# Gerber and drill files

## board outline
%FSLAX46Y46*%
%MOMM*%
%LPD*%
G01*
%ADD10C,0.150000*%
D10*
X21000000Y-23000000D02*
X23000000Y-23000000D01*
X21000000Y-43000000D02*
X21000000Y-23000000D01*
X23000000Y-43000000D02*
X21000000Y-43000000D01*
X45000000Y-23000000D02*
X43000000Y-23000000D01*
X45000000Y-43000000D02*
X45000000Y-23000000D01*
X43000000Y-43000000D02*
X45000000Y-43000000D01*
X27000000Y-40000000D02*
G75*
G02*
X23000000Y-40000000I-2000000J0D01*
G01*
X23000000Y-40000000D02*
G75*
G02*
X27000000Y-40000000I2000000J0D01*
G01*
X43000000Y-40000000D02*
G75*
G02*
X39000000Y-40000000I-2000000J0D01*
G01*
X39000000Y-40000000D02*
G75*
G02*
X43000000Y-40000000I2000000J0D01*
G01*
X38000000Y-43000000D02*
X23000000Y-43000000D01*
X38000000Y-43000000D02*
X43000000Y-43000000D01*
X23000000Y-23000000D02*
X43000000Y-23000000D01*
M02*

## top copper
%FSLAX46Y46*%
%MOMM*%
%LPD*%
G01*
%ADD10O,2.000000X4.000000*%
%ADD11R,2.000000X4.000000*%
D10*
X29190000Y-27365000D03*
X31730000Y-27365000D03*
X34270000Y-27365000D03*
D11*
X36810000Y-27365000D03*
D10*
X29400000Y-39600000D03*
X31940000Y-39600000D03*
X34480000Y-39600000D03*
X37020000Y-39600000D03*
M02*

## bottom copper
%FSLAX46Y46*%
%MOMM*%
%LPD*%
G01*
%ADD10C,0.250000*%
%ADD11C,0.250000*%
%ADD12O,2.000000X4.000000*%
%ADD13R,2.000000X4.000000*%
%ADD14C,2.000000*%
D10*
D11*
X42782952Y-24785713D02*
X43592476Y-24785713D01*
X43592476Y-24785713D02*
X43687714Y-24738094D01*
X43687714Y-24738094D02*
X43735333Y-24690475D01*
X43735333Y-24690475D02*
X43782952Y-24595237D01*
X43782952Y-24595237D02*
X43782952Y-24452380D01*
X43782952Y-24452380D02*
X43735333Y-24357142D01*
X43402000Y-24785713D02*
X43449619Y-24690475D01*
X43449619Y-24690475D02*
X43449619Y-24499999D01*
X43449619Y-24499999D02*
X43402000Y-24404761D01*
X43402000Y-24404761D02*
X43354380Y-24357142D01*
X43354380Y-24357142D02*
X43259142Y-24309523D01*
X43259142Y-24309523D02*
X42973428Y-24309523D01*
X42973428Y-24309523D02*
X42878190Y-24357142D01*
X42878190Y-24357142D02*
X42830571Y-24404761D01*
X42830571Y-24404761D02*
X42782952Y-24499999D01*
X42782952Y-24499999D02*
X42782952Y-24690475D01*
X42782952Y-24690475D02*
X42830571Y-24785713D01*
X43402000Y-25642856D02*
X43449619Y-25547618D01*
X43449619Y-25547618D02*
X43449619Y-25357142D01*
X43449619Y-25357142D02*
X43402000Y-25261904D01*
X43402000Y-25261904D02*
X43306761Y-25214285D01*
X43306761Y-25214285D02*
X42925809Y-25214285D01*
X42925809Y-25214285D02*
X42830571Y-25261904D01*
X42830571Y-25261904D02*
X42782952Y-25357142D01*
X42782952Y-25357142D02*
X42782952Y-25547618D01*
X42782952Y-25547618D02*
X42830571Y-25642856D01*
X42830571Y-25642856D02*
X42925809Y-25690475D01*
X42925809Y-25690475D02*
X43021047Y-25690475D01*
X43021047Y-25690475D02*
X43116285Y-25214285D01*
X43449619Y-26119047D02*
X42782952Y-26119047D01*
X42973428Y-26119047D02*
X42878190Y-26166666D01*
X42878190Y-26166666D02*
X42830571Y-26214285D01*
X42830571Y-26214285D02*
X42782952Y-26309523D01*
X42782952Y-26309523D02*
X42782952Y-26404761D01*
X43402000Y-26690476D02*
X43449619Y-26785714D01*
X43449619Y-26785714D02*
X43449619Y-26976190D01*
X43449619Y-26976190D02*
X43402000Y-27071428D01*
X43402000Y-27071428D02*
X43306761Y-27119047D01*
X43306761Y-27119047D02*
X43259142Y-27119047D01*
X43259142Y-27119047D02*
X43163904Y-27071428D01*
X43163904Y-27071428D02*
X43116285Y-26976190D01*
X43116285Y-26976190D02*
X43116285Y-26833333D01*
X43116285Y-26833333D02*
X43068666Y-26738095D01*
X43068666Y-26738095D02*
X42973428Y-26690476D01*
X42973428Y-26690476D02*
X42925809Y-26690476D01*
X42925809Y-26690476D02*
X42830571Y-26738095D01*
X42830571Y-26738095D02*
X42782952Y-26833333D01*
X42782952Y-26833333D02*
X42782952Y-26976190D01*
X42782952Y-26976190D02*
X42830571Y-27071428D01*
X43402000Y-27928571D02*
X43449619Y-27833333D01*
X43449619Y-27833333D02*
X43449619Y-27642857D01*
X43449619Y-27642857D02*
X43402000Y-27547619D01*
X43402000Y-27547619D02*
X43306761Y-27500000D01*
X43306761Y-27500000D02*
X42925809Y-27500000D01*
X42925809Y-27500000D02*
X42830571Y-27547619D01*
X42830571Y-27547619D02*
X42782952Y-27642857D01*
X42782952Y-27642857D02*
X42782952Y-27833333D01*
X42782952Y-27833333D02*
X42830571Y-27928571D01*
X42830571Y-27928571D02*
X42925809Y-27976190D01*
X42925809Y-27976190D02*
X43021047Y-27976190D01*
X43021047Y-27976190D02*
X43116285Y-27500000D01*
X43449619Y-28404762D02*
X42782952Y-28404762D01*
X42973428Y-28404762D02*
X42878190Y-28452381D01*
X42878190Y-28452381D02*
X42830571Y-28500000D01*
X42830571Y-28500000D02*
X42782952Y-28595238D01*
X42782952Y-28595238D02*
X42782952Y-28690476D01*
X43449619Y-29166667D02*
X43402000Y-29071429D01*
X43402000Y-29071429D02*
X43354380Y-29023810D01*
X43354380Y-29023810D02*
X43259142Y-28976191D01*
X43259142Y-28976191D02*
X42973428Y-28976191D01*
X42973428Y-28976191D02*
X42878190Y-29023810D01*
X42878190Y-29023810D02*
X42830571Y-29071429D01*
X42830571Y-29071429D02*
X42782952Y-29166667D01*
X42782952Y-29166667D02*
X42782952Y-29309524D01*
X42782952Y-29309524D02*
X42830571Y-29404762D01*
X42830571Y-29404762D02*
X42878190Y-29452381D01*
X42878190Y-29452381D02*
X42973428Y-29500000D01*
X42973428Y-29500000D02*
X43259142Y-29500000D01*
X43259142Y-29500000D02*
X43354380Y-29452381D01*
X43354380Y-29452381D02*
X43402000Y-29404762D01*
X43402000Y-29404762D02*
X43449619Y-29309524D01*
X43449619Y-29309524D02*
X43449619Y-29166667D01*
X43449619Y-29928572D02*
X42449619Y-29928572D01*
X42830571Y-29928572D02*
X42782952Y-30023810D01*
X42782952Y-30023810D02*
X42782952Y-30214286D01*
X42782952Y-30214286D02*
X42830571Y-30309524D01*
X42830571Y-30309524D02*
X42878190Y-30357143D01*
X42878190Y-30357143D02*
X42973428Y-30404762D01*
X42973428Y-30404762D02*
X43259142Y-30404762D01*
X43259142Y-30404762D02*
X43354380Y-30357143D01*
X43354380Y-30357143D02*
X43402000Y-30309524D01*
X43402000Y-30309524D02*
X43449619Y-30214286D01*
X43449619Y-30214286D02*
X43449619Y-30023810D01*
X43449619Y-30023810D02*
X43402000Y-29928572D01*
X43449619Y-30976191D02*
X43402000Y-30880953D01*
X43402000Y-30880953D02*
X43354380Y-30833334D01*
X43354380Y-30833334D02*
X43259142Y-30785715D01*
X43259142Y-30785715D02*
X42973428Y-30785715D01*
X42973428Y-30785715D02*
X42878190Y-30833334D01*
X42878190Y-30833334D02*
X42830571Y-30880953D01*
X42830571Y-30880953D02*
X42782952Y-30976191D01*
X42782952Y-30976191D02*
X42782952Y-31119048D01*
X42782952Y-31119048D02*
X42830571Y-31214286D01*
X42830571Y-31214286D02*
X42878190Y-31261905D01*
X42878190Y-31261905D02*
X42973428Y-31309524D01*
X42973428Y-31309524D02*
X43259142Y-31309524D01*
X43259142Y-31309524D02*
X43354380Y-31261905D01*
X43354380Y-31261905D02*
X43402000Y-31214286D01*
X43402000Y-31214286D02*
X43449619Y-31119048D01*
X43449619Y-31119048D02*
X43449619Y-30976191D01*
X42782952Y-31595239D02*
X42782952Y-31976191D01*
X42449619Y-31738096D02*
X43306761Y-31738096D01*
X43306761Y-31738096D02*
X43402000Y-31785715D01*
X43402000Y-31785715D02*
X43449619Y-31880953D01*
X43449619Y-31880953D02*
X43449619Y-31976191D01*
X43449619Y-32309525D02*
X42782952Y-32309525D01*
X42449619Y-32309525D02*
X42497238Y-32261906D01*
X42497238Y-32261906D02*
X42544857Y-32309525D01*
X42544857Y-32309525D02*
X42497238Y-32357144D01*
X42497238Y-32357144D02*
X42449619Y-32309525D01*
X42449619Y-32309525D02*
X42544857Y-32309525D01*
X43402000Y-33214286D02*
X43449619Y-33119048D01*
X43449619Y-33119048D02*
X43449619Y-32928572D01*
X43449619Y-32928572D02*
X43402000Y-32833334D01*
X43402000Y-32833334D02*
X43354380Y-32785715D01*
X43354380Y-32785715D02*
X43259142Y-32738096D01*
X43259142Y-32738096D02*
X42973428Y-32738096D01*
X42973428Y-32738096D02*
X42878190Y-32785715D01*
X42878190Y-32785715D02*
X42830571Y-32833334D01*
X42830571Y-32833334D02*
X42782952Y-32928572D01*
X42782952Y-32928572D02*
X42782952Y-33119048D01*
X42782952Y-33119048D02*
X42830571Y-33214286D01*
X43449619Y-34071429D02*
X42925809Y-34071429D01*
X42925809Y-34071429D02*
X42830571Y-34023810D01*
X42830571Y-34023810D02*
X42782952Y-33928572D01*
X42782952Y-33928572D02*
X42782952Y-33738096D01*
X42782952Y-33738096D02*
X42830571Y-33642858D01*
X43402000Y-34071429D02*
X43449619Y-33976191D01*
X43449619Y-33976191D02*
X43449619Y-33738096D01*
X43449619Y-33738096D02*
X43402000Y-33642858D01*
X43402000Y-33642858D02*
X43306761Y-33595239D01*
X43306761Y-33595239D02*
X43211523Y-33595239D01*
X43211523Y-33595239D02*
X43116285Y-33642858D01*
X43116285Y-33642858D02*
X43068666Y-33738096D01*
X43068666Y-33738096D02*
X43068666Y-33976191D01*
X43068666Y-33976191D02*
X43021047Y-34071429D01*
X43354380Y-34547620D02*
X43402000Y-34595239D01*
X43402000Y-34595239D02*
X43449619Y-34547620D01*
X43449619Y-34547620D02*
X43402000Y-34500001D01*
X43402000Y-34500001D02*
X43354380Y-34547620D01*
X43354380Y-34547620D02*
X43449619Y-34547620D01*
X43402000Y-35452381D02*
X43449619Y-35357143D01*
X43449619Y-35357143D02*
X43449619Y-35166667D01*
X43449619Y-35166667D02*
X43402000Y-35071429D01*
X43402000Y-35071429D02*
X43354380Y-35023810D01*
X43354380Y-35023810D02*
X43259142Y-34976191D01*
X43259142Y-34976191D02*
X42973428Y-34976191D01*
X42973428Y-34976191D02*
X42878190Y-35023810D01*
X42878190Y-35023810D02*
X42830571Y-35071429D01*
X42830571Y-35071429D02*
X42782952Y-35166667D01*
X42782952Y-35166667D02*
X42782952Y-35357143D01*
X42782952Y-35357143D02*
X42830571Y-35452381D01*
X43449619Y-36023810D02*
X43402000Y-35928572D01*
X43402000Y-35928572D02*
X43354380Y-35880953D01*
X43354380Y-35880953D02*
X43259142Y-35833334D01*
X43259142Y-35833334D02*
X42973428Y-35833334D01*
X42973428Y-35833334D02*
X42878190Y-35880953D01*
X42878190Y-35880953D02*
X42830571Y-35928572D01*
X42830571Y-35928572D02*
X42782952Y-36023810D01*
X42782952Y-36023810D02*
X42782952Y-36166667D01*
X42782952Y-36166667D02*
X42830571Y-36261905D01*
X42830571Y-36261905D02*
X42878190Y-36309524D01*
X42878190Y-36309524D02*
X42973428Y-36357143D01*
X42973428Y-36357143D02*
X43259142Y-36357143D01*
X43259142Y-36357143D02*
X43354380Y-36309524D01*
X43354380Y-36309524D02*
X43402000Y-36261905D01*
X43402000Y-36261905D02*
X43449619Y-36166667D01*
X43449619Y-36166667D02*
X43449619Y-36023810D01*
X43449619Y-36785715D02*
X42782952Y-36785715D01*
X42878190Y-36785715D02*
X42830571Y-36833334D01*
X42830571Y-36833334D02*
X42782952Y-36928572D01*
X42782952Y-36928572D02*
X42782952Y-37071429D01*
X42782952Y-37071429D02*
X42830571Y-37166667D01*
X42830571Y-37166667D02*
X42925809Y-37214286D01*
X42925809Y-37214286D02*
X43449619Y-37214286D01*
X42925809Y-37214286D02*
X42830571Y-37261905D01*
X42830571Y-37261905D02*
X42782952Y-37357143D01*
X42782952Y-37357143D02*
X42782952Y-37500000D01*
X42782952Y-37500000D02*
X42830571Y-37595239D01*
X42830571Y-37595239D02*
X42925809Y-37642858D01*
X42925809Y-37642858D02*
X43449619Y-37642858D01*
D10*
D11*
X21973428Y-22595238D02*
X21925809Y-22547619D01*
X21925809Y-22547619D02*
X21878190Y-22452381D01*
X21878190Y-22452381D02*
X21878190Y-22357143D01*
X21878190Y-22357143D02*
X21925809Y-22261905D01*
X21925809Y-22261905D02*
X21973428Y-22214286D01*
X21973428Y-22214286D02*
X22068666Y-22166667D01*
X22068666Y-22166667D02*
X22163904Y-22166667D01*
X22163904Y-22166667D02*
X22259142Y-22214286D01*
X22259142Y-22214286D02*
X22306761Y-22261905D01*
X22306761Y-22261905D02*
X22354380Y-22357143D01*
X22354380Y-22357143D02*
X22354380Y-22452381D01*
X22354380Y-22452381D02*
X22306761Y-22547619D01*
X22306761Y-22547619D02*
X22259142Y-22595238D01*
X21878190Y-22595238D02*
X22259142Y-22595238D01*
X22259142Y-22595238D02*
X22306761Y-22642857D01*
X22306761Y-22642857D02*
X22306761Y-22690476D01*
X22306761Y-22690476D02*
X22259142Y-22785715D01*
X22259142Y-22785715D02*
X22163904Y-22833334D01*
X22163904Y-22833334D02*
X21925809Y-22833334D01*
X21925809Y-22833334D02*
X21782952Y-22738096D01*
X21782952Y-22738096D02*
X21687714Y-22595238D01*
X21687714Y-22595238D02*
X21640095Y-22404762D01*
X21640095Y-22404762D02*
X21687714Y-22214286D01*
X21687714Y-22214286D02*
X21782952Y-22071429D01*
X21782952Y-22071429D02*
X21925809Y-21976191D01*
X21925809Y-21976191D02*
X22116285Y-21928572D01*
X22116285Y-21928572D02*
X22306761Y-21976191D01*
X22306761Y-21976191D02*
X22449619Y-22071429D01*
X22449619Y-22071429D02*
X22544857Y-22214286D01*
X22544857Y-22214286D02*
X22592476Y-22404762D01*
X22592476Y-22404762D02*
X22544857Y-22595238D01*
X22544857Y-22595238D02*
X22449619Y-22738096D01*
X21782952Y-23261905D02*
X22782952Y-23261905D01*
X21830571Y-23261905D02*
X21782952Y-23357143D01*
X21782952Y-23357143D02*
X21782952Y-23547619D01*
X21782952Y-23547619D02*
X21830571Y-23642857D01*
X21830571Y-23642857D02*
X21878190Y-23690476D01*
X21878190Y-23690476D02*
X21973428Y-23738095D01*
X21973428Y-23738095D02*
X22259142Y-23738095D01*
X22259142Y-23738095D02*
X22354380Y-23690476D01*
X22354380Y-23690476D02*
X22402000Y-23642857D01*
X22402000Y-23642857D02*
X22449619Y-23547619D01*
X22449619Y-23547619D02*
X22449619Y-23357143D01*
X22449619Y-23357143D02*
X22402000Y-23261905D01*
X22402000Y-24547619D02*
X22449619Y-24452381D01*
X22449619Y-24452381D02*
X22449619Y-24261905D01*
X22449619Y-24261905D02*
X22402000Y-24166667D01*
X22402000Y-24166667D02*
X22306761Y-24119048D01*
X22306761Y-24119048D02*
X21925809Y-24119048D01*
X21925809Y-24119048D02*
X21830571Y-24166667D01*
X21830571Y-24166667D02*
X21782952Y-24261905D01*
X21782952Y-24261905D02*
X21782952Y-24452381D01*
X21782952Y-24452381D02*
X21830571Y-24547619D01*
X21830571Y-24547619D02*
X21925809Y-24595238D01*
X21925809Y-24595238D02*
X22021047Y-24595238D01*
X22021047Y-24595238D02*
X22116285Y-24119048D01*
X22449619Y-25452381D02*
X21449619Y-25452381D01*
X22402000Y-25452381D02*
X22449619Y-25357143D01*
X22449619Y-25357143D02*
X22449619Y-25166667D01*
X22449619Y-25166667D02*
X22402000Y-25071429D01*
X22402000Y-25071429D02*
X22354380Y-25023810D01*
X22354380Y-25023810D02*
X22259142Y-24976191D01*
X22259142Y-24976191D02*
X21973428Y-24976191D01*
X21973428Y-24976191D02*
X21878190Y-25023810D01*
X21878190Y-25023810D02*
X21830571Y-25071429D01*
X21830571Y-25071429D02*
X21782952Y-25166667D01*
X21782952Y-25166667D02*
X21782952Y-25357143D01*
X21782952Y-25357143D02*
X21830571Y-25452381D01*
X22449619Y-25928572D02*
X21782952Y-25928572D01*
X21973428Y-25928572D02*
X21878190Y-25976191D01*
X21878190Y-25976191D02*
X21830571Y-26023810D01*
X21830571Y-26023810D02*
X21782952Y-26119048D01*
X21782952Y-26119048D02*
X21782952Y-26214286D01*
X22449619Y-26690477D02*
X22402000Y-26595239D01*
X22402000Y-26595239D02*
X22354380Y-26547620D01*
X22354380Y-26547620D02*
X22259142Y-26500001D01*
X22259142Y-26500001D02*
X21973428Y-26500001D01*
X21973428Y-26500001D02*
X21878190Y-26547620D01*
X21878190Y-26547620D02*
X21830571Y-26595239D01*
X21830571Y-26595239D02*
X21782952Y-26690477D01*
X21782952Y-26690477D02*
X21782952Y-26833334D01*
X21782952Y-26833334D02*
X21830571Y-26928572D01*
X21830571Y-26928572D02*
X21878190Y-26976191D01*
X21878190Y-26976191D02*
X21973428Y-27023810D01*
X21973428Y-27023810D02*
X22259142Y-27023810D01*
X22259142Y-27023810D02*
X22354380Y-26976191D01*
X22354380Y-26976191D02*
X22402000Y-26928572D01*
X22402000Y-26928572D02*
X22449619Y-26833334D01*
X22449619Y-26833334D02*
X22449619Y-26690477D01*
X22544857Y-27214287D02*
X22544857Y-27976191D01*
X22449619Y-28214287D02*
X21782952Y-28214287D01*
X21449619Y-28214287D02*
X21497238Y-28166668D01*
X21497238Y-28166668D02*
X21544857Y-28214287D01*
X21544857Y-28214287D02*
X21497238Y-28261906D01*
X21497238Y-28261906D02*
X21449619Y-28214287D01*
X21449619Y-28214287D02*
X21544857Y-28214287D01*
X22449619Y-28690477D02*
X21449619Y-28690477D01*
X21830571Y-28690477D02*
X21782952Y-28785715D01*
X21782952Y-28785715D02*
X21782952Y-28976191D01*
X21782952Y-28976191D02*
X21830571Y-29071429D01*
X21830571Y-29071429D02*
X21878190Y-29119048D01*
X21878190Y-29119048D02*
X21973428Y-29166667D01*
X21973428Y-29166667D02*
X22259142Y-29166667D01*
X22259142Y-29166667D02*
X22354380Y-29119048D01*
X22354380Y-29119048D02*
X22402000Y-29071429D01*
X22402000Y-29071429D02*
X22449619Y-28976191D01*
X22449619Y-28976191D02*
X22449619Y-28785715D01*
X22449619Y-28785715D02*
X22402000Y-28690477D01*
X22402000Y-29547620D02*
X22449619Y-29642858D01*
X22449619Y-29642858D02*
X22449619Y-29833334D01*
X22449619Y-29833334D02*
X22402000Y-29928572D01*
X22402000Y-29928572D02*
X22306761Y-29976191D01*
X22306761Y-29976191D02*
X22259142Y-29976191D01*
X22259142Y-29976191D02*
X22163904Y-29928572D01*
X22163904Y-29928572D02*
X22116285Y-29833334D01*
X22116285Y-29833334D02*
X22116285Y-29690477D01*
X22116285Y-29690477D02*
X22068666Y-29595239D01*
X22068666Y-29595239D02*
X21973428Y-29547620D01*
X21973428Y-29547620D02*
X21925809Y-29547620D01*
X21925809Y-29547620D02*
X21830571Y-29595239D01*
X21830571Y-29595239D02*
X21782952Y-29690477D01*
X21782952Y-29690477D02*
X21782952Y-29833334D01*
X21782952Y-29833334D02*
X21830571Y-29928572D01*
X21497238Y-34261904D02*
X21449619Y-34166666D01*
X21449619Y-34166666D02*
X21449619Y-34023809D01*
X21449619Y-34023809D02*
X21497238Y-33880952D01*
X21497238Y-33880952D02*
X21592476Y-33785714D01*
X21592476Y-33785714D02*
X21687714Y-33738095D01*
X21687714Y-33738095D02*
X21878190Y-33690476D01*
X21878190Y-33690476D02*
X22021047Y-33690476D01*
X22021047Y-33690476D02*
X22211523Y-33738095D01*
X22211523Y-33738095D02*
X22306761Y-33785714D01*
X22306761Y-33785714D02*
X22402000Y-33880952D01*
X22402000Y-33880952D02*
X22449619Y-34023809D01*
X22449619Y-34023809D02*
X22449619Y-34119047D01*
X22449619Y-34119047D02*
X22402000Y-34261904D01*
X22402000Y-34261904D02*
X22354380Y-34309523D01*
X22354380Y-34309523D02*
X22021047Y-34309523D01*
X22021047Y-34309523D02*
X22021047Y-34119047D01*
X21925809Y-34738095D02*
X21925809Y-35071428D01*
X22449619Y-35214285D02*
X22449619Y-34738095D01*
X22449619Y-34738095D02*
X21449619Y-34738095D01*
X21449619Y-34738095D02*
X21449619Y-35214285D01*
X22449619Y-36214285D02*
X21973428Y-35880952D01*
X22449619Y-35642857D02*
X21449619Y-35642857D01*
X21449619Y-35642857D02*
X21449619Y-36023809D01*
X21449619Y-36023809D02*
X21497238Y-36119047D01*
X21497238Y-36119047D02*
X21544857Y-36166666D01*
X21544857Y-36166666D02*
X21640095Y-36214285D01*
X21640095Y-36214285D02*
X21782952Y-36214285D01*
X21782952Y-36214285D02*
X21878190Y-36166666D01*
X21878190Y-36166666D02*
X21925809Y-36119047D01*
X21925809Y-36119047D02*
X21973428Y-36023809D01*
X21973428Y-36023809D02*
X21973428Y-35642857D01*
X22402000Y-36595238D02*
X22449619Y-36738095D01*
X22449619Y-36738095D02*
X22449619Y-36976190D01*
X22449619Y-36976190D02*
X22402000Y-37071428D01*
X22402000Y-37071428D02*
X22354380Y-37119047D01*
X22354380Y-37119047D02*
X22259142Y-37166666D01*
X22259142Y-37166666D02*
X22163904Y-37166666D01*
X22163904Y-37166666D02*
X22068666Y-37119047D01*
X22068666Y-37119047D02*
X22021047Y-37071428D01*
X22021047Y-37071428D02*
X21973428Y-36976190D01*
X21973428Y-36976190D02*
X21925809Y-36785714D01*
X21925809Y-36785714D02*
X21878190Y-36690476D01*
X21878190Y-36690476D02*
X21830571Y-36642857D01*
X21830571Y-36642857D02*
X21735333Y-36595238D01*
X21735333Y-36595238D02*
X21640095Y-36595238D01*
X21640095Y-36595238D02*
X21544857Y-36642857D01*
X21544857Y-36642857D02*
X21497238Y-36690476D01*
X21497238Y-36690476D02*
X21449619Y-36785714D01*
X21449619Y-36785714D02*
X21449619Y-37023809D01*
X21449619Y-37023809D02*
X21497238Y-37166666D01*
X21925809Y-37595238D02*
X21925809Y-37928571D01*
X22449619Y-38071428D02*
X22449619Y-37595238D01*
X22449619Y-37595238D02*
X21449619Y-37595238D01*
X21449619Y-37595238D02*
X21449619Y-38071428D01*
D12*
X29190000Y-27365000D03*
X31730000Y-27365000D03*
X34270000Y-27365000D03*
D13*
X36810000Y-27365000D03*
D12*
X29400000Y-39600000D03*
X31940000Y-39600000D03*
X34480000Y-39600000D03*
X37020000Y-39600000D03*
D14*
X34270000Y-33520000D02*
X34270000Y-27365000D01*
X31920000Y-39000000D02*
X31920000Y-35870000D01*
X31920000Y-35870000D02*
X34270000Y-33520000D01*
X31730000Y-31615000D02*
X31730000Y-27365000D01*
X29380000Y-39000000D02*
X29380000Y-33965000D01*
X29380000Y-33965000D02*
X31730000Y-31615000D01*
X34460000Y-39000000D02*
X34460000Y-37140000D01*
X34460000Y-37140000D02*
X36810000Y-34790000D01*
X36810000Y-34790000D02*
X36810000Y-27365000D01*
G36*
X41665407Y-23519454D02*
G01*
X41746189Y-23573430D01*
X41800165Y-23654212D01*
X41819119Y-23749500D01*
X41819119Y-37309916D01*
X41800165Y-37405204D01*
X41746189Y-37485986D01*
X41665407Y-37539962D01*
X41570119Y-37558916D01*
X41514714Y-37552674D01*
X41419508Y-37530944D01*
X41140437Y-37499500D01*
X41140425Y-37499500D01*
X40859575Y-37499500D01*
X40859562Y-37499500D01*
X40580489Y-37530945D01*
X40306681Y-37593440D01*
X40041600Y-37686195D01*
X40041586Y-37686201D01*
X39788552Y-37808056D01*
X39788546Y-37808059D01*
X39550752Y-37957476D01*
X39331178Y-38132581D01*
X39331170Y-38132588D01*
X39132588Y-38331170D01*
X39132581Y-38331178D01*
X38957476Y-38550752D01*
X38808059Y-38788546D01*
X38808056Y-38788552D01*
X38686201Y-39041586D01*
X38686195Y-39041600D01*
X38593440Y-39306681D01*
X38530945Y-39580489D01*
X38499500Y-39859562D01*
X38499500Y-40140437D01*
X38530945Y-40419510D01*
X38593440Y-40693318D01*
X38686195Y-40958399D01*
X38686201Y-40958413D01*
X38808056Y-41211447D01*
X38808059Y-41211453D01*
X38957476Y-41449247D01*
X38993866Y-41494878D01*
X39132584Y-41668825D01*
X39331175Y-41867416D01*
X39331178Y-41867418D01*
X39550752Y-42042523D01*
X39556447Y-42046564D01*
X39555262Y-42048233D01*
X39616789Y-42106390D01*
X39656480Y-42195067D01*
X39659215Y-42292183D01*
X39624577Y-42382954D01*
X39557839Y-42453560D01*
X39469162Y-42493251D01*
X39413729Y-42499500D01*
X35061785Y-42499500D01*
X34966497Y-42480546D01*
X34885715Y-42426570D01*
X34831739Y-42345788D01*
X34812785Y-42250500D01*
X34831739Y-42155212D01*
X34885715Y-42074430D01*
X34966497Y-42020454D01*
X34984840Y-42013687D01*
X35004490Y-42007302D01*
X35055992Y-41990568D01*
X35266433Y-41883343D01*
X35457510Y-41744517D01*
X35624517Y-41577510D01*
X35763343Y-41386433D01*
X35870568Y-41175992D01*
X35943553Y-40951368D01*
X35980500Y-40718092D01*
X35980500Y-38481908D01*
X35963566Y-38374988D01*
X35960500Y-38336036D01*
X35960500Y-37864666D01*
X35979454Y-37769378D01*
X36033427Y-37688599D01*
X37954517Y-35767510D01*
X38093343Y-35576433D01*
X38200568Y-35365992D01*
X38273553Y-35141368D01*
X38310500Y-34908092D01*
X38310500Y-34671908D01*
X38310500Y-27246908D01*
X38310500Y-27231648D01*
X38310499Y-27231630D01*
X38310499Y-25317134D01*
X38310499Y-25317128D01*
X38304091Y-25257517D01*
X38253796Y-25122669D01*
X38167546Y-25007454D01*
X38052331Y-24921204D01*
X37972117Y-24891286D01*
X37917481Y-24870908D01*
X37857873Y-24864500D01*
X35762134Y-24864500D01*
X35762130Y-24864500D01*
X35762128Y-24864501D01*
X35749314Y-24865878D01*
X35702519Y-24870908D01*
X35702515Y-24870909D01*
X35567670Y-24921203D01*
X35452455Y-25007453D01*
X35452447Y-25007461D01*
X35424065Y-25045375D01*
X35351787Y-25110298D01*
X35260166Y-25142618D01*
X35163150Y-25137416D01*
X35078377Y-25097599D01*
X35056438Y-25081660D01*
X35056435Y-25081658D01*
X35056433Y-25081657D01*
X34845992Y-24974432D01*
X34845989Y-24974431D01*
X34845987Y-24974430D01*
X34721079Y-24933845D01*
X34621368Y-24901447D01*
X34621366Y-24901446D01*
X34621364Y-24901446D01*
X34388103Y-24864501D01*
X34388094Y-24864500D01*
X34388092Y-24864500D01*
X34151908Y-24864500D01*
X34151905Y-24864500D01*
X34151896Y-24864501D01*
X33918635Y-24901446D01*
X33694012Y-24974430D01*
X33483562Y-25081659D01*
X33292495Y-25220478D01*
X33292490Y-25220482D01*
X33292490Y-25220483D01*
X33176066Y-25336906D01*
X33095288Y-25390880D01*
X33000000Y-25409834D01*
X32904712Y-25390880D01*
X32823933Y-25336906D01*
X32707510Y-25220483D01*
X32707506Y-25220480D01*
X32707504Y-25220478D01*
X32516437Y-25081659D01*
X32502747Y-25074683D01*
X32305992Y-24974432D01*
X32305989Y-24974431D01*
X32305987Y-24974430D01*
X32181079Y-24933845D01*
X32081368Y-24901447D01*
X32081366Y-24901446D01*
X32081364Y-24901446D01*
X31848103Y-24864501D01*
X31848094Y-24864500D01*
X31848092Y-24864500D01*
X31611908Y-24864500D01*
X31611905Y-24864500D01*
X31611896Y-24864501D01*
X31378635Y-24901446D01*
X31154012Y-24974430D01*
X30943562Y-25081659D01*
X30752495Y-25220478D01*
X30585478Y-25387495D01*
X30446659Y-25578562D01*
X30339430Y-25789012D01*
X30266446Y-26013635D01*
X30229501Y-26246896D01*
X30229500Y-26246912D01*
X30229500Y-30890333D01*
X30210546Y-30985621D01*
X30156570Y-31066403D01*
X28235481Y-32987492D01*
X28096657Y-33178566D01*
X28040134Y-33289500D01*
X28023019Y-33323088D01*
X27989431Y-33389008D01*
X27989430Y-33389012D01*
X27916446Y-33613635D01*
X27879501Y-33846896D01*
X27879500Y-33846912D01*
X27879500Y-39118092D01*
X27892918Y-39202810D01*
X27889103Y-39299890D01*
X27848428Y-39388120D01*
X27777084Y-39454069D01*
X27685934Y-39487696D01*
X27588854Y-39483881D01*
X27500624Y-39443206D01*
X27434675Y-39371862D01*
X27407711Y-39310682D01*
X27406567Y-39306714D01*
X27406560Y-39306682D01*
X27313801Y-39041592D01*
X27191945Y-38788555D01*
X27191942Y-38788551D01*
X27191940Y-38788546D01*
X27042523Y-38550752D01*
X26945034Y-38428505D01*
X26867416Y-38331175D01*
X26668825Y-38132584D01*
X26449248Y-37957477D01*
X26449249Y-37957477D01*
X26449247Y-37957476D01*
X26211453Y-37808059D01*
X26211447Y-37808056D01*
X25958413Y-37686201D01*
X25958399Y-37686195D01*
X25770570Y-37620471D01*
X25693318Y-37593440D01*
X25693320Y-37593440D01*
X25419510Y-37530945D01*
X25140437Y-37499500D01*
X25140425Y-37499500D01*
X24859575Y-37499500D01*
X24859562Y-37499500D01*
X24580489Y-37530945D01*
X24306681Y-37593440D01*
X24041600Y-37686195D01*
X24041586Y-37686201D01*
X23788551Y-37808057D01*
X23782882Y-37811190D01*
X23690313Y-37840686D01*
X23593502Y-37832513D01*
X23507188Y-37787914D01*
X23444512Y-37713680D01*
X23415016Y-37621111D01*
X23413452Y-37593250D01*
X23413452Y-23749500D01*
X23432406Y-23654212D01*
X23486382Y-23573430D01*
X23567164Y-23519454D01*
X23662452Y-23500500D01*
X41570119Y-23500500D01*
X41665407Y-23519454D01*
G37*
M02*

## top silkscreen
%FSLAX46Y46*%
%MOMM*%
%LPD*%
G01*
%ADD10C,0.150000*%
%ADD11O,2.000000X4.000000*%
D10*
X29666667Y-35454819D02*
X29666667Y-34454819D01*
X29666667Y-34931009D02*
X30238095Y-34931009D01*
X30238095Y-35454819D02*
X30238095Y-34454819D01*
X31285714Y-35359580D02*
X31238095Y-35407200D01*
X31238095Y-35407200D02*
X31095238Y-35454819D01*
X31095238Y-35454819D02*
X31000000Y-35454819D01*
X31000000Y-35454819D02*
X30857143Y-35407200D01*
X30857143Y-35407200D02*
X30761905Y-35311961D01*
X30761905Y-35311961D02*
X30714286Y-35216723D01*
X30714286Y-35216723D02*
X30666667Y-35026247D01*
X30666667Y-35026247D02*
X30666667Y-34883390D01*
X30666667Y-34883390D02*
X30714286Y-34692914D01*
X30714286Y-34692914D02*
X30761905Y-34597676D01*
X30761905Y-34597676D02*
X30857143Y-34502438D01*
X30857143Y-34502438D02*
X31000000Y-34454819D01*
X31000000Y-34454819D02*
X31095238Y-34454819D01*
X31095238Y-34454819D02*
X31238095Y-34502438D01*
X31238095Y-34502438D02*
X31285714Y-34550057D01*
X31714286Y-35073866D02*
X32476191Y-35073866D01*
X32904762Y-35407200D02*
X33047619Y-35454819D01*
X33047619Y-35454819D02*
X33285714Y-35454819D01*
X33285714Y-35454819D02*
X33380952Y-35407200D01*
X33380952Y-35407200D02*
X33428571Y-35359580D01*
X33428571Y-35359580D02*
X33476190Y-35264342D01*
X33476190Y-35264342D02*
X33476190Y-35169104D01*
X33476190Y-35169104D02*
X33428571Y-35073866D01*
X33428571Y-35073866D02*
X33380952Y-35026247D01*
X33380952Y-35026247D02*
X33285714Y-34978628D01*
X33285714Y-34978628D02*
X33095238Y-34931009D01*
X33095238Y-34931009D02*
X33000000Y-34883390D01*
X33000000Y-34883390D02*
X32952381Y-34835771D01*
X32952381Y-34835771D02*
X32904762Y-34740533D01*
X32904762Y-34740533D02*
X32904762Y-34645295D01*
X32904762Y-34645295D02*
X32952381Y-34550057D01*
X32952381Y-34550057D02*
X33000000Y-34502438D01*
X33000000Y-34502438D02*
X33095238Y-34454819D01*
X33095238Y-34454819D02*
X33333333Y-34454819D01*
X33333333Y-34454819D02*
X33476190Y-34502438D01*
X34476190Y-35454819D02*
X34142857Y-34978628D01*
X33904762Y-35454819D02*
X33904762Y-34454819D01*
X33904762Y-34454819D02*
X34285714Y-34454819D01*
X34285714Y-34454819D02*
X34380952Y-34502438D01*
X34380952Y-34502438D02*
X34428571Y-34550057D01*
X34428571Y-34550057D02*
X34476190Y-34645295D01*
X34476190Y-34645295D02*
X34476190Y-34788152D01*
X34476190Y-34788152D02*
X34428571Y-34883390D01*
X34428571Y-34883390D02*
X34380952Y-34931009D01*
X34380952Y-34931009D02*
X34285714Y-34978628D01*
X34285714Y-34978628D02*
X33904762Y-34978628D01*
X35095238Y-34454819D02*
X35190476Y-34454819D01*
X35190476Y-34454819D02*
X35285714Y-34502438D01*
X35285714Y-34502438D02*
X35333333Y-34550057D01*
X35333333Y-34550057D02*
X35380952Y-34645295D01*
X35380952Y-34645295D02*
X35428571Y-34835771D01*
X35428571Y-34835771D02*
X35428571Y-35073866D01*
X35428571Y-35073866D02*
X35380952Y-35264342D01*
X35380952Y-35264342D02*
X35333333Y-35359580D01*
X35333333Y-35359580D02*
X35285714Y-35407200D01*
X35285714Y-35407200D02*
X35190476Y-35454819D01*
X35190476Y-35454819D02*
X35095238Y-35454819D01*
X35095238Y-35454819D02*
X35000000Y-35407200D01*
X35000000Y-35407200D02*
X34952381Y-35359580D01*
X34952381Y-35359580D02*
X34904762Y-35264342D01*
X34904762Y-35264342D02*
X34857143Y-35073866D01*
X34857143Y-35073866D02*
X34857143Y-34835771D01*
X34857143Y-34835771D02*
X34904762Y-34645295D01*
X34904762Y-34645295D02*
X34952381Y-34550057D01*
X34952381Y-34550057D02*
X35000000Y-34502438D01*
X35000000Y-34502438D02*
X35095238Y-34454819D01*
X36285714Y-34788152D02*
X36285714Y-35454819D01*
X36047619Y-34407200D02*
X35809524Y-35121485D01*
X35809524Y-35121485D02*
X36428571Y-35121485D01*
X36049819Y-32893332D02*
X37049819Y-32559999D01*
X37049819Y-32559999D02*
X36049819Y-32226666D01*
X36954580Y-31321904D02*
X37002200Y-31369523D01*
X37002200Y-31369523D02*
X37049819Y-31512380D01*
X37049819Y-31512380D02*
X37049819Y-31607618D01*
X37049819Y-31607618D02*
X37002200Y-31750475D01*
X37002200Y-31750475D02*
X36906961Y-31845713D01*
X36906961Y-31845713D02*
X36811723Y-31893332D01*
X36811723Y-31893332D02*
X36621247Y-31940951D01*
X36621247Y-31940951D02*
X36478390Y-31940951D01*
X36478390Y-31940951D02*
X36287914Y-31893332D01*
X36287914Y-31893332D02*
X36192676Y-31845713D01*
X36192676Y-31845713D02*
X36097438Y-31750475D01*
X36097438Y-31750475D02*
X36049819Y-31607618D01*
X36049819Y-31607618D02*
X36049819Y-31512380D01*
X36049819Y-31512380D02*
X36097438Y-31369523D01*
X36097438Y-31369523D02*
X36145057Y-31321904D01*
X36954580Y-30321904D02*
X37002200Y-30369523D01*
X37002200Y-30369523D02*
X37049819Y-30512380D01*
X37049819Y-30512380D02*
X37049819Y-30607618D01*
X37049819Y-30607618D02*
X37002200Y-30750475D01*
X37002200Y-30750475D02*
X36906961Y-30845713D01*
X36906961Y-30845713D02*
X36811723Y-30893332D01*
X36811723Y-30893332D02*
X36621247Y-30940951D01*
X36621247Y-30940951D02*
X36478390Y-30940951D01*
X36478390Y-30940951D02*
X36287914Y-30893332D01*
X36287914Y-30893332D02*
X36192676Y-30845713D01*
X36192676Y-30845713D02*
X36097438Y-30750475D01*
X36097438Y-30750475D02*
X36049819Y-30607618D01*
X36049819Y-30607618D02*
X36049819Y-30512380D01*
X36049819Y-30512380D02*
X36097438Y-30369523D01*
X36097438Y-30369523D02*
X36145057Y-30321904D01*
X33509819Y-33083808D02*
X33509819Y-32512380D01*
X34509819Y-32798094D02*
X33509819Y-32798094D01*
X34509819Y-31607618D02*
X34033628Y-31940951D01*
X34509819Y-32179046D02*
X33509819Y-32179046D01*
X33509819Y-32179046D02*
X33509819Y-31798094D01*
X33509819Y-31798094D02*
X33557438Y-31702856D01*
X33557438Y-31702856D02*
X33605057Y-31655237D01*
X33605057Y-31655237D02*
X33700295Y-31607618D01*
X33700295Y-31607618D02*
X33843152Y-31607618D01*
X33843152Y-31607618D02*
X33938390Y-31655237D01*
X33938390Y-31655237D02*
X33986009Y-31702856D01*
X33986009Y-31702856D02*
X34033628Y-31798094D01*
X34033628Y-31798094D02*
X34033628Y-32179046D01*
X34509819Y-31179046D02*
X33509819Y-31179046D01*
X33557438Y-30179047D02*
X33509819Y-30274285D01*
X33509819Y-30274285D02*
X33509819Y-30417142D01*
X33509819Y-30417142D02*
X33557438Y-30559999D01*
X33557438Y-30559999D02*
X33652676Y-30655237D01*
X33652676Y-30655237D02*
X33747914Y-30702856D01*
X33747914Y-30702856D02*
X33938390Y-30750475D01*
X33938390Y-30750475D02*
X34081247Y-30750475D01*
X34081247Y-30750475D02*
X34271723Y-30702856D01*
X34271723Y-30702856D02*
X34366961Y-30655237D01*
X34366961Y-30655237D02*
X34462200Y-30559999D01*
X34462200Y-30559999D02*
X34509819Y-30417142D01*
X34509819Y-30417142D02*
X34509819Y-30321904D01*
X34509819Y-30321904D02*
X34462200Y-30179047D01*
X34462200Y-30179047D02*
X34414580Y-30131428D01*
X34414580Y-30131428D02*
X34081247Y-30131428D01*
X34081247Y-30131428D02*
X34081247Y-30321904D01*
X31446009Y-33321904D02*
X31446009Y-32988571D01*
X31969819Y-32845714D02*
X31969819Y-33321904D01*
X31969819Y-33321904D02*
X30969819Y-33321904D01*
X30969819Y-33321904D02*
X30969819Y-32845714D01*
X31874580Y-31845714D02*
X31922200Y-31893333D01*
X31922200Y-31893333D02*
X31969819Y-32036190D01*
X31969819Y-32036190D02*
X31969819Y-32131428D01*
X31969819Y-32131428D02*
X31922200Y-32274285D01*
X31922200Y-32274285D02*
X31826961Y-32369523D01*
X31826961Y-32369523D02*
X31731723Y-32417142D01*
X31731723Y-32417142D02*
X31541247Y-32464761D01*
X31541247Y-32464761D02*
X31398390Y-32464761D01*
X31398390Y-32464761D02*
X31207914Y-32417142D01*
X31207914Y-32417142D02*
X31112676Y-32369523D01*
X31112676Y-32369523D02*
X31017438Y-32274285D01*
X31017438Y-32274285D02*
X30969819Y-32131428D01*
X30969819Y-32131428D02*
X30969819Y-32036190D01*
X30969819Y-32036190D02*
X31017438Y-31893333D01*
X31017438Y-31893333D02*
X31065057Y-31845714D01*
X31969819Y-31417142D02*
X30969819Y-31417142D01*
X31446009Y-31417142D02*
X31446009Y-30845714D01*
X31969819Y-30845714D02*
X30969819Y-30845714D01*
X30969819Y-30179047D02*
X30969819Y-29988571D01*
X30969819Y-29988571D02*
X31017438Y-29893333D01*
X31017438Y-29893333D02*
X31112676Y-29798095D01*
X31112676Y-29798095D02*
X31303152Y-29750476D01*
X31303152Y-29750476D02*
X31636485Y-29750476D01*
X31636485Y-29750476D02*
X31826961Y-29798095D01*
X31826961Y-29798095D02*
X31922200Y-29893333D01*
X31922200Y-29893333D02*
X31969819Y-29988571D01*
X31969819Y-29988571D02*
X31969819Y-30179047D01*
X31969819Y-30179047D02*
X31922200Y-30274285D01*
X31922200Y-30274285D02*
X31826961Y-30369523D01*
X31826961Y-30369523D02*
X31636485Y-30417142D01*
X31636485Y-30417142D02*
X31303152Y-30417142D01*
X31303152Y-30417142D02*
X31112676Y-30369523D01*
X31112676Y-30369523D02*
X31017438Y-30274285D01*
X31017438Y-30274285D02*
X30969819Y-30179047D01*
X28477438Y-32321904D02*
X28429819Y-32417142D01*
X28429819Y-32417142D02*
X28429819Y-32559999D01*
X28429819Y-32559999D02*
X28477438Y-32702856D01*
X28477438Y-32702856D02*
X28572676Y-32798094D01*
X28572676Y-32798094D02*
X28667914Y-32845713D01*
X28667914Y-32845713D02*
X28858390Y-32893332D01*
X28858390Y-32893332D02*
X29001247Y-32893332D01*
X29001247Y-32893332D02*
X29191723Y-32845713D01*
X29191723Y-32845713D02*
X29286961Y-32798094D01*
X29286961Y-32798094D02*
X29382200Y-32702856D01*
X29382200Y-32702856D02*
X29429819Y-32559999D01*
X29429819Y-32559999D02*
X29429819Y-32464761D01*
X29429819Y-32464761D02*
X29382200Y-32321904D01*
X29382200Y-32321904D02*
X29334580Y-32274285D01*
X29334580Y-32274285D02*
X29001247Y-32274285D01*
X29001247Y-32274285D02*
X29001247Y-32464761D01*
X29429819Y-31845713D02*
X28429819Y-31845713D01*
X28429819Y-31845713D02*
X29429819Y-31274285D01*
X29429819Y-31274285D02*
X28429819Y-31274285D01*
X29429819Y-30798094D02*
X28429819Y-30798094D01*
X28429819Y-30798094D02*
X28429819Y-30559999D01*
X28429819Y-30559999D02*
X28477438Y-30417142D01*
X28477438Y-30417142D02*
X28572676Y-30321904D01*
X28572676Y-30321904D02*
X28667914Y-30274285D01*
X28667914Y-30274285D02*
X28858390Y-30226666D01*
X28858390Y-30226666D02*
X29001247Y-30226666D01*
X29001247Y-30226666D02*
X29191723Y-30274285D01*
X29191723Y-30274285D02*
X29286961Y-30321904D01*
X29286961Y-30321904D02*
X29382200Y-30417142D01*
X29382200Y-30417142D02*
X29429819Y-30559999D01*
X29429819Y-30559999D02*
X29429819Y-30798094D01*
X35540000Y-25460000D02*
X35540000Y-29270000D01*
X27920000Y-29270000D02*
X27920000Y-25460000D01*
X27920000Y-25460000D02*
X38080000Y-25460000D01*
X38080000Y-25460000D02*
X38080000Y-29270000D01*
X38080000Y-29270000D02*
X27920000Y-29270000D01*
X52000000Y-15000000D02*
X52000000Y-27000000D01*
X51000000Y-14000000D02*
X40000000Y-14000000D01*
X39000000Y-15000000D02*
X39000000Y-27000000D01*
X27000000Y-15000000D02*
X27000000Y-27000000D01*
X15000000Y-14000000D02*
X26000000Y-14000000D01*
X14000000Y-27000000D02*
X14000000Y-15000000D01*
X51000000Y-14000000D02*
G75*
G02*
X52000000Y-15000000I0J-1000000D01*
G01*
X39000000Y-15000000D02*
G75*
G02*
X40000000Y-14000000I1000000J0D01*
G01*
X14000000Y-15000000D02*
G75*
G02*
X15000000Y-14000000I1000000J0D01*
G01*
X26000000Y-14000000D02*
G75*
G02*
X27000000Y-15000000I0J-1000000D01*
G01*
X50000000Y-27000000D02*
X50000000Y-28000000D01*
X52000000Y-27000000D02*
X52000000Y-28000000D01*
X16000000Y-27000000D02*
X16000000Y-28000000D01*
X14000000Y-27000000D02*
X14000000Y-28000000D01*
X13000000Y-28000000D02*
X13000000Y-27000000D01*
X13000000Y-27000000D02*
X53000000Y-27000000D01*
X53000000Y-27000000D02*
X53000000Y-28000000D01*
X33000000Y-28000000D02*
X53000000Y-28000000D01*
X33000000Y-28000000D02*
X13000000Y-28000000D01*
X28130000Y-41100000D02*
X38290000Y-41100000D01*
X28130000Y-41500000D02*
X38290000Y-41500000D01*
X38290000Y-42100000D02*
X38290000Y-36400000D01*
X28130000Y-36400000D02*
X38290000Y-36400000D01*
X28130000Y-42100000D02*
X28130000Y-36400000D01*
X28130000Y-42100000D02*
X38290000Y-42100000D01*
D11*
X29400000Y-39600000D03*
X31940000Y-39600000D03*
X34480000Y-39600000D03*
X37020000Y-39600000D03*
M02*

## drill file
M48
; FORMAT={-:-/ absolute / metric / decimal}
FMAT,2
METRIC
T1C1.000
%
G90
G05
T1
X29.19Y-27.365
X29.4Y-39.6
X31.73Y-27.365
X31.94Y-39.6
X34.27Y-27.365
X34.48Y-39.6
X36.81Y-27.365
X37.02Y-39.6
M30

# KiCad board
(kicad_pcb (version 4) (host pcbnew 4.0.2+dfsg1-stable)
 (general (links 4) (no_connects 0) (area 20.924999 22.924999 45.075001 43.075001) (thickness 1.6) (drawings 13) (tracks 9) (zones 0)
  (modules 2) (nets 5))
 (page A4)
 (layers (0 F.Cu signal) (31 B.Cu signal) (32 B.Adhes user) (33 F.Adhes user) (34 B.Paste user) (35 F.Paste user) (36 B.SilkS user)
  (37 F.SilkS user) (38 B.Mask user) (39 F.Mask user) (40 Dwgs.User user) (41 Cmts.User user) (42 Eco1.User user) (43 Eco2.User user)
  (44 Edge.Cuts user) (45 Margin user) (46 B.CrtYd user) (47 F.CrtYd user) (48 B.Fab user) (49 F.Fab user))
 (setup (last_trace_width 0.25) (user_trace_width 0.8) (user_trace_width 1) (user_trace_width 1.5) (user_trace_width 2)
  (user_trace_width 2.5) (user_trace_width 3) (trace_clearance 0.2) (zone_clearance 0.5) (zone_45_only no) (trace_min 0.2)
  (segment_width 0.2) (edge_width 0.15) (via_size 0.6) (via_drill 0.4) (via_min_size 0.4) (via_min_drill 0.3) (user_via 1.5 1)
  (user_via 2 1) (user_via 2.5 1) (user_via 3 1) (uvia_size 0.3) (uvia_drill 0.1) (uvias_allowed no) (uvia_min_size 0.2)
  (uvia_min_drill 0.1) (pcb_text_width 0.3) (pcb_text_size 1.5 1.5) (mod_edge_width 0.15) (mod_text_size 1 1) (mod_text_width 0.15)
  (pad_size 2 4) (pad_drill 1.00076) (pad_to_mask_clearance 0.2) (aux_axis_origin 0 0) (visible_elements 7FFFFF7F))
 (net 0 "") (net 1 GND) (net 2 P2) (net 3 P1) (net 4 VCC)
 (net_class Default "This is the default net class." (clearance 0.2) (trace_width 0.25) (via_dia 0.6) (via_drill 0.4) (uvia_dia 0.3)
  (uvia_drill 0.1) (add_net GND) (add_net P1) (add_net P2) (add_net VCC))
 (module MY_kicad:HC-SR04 (layer F.Cu) (at 33 28)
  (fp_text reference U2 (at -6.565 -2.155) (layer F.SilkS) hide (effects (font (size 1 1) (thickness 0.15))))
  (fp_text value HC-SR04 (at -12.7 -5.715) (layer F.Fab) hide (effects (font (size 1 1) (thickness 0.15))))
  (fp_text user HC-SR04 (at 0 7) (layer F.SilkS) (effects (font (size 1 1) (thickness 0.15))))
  (fp_line (start 2.54 -2.54) (end 2.54 1.27) (layer F.SilkS) (width 0.15))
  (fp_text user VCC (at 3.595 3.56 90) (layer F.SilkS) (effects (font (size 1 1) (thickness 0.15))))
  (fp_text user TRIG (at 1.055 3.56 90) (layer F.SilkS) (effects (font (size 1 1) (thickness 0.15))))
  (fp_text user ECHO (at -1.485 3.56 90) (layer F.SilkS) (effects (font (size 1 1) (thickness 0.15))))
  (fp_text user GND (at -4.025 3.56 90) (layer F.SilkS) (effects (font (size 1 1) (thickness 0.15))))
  (fp_line (start -5.08 1.27) (end -5.08 -2.54) (layer F.SilkS) (width 0.15))
  (fp_line (start -5.08 -2.54) (end 5.08 -2.54) (layer F.SilkS) (width 0.15))
  (fp_line (start 5.08 -2.54) (end 5.08 1.27) (layer F.SilkS) (width 0.15))
  (fp_line (start 5.08 1.27) (end -5.08 1.27) (layer F.SilkS) (width 0.15))
  (fp_line (start 19 -13) (end 19 -1) (layer F.SilkS) (width 0.15))
  (fp_line (start 18 -14) (end 7 -14) (layer F.SilkS) (width 0.15))
  (fp_line (start 6 -13) (end 6 -1) (layer F.SilkS) (width 0.15))
  (fp_line (start -6 -13) (end -6 -1) (layer F.SilkS) (width 0.15))
  (fp_line (start -18 -14) (end -7 -14) (layer F.SilkS) (width 0.15))
  (fp_line (start -19 -1) (end -19 -13) (layer F.SilkS) (width 0.15))
  (fp_arc (start 18 -13) (end 18 -14) (angle 90) (layer F.SilkS) (width 0.15))
  (fp_arc (start 7 -13) (end 6 -13) (angle 90) (layer F.SilkS) (width 0.15))
  (fp_arc (start -18 -13) (end -19 -13) (angle 90) (layer F.SilkS) (width 0.15))
  (fp_arc (start -7 -13) (end -7 -14) (angle 90) (layer F.SilkS) (width 0.15))
  (fp_line (start 17 -1) (end 17 0) (layer F.SilkS) (width 0.15))
  (fp_line (start 19 -1) (end 19 0) (layer F.SilkS) (width 0.15))
  (fp_line (start -17 -1) (end -17 0) (layer F.SilkS) (width 0.15))
  (fp_line (start -19 -1) (end -19 0) (layer F.SilkS) (width 0.15))
  (fp_line (start -20 0) (end -20 -1) (layer F.SilkS) (width 0.15))
  (fp_line (start -20 -1) (end 20 -1) (layer F.SilkS) (width 0.15))
  (fp_line (start 20 -1) (end 20 0) (layer F.SilkS) (width 0.15))
  (fp_line (start 0 0) (end 20 0) (layer F.SilkS) (width 0.15))
  (fp_line (start 0 0) (end -20 0) (layer F.SilkS) (width 0.15))
  (pad 4 thru_hole oval (at -3.81 -0.635) (size 2 4) (drill 1) (layers *.Cu *.Mask) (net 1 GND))
  (pad 3 thru_hole oval (at -1.27 -0.635) (size 2 4) (drill 1) (layers *.Cu *.Mask) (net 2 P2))
  (pad 2 thru_hole oval (at 1.27 -0.635) (size 2 4) (drill 1) (layers *.Cu *.Mask) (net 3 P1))
  (pad 1 thru_hole rect (at 3.81 -0.635) (size 2 4) (drill 1) (layers *.Cu *.Mask) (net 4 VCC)))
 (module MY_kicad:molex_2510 (layer F.Cu) (at 29.4 39.6)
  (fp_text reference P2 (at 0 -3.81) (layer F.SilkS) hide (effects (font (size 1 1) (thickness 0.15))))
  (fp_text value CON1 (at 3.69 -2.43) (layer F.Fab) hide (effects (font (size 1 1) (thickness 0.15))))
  (fp_line (start -1.27 1.5) (end 8.89 1.5) (layer F.SilkS) (width 0.15))
  (fp_line (start -1.27 1.9) (end 8.89 1.9) (layer F.SilkS) (width 0.15))
  (fp_line (start 8.89 2.5) (end 8.89 -3.2) (layer F.SilkS) (width 0.15))
  (fp_line (start -1.27 -3.2) (end 8.89 -3.2) (layer F.SilkS) (width 0.15))
  (fp_line (start -1.27 2.5) (end -1.27 -3.2) (layer F.SilkS) (width 0.15))
  (fp_line (start -1.27 2.5) (end 8.89 2.5) (layer F.SilkS) (width 0.15))
  (pad 1 thru_hole oval (at 0 0) (size 2 4) (drill 1) (layers *.Cu *.Mask F.SilkS) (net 2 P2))
  (pad 2 thru_hole oval (at 2.54 0) (size 2 4) (drill 1) (layers *.Cu *.Mask F.SilkS) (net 3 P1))
  (pad 3 thru_hole oval (at 5.08 0) (size 2 4) (drill 1) (layers *.Cu *.Mask F.SilkS) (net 4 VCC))
  (pad 4 thru_hole oval (at 7.62 0) (size 2 4) (drill 1) (layers *.Cu *.Mask F.SilkS) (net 1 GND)))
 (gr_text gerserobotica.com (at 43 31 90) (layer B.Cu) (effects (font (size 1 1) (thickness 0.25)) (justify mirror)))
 (gr_line (start 21 23) (end 23 23) (angle 90) (layer Edge.Cuts) (width 0.15))
 (gr_line (start 21 43) (end 21 23) (angle 90) (layer Edge.Cuts) (width 0.15))
 (gr_line (start 23 43) (end 21 43) (angle 90) (layer Edge.Cuts) (width 0.15))
 (gr_line (start 45 23) (end 43 23) (angle 90) (layer Edge.Cuts) (width 0.15))
 (gr_line (start 45 43) (end 45 23) (angle 90) (layer Edge.Cuts) (width 0.15))
 (gr_line (start 43 43) (end 45 43) (angle 90) (layer Edge.Cuts) (width 0.15))
 (gr_circle (center 25 40) (end 27 40) (layer Edge.Cuts) (width 0.15))
 (gr_circle (center 41 40) (end 43 40) (layer Edge.Cuts) (width 0.15))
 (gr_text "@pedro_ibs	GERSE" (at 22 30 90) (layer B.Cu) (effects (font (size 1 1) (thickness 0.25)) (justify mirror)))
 (gr_line (start 38 43) (end 23 43) (angle 90) (layer Edge.Cuts) (width 0.15))
 (gr_line (start 38 43) (end 43 43) (angle 90) (layer Edge.Cuts) (width 0.15))
 (gr_line (start 23 23) (end 43 23) (angle 90) (layer Edge.Cuts) (width 0.15))
 (segment (start 34.27 33.52) (end 34.27 27.365) (width 2) (layer B.Cu) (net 3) (status 20))
 (segment (start 31.92 39) (end 31.92 35.87) (width 2) (layer B.Cu) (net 3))
 (segment (start 31.92 35.87) (end 34.27 33.52) (width 2) (layer B.Cu) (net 3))
 (segment (start 31.73 31.615) (end 31.73 27.365) (width 2) (layer B.Cu) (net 2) (status 20))
 (segment (start 29.38 39) (end 29.38 33.965) (width 2) (layer B.Cu) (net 2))
 (segment (start 29.38 33.965) (end 31.73 31.615) (width 2) (layer B.Cu) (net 2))
 (segment (start 34.46 39) (end 34.46 37.14) (width 2) (layer B.Cu) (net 4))
 (segment (start 34.46 37.14) (end 36.81 34.79) (width 2) (layer B.Cu) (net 4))
 (segment (start 36.81 34.79) (end 36.81 27.365) (width 2) (layer B.Cu) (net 4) (status 20))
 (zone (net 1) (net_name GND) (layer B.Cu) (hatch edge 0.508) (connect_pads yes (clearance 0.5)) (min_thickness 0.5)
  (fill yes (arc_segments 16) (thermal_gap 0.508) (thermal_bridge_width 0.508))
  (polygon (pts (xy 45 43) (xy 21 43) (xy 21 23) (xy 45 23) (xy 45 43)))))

